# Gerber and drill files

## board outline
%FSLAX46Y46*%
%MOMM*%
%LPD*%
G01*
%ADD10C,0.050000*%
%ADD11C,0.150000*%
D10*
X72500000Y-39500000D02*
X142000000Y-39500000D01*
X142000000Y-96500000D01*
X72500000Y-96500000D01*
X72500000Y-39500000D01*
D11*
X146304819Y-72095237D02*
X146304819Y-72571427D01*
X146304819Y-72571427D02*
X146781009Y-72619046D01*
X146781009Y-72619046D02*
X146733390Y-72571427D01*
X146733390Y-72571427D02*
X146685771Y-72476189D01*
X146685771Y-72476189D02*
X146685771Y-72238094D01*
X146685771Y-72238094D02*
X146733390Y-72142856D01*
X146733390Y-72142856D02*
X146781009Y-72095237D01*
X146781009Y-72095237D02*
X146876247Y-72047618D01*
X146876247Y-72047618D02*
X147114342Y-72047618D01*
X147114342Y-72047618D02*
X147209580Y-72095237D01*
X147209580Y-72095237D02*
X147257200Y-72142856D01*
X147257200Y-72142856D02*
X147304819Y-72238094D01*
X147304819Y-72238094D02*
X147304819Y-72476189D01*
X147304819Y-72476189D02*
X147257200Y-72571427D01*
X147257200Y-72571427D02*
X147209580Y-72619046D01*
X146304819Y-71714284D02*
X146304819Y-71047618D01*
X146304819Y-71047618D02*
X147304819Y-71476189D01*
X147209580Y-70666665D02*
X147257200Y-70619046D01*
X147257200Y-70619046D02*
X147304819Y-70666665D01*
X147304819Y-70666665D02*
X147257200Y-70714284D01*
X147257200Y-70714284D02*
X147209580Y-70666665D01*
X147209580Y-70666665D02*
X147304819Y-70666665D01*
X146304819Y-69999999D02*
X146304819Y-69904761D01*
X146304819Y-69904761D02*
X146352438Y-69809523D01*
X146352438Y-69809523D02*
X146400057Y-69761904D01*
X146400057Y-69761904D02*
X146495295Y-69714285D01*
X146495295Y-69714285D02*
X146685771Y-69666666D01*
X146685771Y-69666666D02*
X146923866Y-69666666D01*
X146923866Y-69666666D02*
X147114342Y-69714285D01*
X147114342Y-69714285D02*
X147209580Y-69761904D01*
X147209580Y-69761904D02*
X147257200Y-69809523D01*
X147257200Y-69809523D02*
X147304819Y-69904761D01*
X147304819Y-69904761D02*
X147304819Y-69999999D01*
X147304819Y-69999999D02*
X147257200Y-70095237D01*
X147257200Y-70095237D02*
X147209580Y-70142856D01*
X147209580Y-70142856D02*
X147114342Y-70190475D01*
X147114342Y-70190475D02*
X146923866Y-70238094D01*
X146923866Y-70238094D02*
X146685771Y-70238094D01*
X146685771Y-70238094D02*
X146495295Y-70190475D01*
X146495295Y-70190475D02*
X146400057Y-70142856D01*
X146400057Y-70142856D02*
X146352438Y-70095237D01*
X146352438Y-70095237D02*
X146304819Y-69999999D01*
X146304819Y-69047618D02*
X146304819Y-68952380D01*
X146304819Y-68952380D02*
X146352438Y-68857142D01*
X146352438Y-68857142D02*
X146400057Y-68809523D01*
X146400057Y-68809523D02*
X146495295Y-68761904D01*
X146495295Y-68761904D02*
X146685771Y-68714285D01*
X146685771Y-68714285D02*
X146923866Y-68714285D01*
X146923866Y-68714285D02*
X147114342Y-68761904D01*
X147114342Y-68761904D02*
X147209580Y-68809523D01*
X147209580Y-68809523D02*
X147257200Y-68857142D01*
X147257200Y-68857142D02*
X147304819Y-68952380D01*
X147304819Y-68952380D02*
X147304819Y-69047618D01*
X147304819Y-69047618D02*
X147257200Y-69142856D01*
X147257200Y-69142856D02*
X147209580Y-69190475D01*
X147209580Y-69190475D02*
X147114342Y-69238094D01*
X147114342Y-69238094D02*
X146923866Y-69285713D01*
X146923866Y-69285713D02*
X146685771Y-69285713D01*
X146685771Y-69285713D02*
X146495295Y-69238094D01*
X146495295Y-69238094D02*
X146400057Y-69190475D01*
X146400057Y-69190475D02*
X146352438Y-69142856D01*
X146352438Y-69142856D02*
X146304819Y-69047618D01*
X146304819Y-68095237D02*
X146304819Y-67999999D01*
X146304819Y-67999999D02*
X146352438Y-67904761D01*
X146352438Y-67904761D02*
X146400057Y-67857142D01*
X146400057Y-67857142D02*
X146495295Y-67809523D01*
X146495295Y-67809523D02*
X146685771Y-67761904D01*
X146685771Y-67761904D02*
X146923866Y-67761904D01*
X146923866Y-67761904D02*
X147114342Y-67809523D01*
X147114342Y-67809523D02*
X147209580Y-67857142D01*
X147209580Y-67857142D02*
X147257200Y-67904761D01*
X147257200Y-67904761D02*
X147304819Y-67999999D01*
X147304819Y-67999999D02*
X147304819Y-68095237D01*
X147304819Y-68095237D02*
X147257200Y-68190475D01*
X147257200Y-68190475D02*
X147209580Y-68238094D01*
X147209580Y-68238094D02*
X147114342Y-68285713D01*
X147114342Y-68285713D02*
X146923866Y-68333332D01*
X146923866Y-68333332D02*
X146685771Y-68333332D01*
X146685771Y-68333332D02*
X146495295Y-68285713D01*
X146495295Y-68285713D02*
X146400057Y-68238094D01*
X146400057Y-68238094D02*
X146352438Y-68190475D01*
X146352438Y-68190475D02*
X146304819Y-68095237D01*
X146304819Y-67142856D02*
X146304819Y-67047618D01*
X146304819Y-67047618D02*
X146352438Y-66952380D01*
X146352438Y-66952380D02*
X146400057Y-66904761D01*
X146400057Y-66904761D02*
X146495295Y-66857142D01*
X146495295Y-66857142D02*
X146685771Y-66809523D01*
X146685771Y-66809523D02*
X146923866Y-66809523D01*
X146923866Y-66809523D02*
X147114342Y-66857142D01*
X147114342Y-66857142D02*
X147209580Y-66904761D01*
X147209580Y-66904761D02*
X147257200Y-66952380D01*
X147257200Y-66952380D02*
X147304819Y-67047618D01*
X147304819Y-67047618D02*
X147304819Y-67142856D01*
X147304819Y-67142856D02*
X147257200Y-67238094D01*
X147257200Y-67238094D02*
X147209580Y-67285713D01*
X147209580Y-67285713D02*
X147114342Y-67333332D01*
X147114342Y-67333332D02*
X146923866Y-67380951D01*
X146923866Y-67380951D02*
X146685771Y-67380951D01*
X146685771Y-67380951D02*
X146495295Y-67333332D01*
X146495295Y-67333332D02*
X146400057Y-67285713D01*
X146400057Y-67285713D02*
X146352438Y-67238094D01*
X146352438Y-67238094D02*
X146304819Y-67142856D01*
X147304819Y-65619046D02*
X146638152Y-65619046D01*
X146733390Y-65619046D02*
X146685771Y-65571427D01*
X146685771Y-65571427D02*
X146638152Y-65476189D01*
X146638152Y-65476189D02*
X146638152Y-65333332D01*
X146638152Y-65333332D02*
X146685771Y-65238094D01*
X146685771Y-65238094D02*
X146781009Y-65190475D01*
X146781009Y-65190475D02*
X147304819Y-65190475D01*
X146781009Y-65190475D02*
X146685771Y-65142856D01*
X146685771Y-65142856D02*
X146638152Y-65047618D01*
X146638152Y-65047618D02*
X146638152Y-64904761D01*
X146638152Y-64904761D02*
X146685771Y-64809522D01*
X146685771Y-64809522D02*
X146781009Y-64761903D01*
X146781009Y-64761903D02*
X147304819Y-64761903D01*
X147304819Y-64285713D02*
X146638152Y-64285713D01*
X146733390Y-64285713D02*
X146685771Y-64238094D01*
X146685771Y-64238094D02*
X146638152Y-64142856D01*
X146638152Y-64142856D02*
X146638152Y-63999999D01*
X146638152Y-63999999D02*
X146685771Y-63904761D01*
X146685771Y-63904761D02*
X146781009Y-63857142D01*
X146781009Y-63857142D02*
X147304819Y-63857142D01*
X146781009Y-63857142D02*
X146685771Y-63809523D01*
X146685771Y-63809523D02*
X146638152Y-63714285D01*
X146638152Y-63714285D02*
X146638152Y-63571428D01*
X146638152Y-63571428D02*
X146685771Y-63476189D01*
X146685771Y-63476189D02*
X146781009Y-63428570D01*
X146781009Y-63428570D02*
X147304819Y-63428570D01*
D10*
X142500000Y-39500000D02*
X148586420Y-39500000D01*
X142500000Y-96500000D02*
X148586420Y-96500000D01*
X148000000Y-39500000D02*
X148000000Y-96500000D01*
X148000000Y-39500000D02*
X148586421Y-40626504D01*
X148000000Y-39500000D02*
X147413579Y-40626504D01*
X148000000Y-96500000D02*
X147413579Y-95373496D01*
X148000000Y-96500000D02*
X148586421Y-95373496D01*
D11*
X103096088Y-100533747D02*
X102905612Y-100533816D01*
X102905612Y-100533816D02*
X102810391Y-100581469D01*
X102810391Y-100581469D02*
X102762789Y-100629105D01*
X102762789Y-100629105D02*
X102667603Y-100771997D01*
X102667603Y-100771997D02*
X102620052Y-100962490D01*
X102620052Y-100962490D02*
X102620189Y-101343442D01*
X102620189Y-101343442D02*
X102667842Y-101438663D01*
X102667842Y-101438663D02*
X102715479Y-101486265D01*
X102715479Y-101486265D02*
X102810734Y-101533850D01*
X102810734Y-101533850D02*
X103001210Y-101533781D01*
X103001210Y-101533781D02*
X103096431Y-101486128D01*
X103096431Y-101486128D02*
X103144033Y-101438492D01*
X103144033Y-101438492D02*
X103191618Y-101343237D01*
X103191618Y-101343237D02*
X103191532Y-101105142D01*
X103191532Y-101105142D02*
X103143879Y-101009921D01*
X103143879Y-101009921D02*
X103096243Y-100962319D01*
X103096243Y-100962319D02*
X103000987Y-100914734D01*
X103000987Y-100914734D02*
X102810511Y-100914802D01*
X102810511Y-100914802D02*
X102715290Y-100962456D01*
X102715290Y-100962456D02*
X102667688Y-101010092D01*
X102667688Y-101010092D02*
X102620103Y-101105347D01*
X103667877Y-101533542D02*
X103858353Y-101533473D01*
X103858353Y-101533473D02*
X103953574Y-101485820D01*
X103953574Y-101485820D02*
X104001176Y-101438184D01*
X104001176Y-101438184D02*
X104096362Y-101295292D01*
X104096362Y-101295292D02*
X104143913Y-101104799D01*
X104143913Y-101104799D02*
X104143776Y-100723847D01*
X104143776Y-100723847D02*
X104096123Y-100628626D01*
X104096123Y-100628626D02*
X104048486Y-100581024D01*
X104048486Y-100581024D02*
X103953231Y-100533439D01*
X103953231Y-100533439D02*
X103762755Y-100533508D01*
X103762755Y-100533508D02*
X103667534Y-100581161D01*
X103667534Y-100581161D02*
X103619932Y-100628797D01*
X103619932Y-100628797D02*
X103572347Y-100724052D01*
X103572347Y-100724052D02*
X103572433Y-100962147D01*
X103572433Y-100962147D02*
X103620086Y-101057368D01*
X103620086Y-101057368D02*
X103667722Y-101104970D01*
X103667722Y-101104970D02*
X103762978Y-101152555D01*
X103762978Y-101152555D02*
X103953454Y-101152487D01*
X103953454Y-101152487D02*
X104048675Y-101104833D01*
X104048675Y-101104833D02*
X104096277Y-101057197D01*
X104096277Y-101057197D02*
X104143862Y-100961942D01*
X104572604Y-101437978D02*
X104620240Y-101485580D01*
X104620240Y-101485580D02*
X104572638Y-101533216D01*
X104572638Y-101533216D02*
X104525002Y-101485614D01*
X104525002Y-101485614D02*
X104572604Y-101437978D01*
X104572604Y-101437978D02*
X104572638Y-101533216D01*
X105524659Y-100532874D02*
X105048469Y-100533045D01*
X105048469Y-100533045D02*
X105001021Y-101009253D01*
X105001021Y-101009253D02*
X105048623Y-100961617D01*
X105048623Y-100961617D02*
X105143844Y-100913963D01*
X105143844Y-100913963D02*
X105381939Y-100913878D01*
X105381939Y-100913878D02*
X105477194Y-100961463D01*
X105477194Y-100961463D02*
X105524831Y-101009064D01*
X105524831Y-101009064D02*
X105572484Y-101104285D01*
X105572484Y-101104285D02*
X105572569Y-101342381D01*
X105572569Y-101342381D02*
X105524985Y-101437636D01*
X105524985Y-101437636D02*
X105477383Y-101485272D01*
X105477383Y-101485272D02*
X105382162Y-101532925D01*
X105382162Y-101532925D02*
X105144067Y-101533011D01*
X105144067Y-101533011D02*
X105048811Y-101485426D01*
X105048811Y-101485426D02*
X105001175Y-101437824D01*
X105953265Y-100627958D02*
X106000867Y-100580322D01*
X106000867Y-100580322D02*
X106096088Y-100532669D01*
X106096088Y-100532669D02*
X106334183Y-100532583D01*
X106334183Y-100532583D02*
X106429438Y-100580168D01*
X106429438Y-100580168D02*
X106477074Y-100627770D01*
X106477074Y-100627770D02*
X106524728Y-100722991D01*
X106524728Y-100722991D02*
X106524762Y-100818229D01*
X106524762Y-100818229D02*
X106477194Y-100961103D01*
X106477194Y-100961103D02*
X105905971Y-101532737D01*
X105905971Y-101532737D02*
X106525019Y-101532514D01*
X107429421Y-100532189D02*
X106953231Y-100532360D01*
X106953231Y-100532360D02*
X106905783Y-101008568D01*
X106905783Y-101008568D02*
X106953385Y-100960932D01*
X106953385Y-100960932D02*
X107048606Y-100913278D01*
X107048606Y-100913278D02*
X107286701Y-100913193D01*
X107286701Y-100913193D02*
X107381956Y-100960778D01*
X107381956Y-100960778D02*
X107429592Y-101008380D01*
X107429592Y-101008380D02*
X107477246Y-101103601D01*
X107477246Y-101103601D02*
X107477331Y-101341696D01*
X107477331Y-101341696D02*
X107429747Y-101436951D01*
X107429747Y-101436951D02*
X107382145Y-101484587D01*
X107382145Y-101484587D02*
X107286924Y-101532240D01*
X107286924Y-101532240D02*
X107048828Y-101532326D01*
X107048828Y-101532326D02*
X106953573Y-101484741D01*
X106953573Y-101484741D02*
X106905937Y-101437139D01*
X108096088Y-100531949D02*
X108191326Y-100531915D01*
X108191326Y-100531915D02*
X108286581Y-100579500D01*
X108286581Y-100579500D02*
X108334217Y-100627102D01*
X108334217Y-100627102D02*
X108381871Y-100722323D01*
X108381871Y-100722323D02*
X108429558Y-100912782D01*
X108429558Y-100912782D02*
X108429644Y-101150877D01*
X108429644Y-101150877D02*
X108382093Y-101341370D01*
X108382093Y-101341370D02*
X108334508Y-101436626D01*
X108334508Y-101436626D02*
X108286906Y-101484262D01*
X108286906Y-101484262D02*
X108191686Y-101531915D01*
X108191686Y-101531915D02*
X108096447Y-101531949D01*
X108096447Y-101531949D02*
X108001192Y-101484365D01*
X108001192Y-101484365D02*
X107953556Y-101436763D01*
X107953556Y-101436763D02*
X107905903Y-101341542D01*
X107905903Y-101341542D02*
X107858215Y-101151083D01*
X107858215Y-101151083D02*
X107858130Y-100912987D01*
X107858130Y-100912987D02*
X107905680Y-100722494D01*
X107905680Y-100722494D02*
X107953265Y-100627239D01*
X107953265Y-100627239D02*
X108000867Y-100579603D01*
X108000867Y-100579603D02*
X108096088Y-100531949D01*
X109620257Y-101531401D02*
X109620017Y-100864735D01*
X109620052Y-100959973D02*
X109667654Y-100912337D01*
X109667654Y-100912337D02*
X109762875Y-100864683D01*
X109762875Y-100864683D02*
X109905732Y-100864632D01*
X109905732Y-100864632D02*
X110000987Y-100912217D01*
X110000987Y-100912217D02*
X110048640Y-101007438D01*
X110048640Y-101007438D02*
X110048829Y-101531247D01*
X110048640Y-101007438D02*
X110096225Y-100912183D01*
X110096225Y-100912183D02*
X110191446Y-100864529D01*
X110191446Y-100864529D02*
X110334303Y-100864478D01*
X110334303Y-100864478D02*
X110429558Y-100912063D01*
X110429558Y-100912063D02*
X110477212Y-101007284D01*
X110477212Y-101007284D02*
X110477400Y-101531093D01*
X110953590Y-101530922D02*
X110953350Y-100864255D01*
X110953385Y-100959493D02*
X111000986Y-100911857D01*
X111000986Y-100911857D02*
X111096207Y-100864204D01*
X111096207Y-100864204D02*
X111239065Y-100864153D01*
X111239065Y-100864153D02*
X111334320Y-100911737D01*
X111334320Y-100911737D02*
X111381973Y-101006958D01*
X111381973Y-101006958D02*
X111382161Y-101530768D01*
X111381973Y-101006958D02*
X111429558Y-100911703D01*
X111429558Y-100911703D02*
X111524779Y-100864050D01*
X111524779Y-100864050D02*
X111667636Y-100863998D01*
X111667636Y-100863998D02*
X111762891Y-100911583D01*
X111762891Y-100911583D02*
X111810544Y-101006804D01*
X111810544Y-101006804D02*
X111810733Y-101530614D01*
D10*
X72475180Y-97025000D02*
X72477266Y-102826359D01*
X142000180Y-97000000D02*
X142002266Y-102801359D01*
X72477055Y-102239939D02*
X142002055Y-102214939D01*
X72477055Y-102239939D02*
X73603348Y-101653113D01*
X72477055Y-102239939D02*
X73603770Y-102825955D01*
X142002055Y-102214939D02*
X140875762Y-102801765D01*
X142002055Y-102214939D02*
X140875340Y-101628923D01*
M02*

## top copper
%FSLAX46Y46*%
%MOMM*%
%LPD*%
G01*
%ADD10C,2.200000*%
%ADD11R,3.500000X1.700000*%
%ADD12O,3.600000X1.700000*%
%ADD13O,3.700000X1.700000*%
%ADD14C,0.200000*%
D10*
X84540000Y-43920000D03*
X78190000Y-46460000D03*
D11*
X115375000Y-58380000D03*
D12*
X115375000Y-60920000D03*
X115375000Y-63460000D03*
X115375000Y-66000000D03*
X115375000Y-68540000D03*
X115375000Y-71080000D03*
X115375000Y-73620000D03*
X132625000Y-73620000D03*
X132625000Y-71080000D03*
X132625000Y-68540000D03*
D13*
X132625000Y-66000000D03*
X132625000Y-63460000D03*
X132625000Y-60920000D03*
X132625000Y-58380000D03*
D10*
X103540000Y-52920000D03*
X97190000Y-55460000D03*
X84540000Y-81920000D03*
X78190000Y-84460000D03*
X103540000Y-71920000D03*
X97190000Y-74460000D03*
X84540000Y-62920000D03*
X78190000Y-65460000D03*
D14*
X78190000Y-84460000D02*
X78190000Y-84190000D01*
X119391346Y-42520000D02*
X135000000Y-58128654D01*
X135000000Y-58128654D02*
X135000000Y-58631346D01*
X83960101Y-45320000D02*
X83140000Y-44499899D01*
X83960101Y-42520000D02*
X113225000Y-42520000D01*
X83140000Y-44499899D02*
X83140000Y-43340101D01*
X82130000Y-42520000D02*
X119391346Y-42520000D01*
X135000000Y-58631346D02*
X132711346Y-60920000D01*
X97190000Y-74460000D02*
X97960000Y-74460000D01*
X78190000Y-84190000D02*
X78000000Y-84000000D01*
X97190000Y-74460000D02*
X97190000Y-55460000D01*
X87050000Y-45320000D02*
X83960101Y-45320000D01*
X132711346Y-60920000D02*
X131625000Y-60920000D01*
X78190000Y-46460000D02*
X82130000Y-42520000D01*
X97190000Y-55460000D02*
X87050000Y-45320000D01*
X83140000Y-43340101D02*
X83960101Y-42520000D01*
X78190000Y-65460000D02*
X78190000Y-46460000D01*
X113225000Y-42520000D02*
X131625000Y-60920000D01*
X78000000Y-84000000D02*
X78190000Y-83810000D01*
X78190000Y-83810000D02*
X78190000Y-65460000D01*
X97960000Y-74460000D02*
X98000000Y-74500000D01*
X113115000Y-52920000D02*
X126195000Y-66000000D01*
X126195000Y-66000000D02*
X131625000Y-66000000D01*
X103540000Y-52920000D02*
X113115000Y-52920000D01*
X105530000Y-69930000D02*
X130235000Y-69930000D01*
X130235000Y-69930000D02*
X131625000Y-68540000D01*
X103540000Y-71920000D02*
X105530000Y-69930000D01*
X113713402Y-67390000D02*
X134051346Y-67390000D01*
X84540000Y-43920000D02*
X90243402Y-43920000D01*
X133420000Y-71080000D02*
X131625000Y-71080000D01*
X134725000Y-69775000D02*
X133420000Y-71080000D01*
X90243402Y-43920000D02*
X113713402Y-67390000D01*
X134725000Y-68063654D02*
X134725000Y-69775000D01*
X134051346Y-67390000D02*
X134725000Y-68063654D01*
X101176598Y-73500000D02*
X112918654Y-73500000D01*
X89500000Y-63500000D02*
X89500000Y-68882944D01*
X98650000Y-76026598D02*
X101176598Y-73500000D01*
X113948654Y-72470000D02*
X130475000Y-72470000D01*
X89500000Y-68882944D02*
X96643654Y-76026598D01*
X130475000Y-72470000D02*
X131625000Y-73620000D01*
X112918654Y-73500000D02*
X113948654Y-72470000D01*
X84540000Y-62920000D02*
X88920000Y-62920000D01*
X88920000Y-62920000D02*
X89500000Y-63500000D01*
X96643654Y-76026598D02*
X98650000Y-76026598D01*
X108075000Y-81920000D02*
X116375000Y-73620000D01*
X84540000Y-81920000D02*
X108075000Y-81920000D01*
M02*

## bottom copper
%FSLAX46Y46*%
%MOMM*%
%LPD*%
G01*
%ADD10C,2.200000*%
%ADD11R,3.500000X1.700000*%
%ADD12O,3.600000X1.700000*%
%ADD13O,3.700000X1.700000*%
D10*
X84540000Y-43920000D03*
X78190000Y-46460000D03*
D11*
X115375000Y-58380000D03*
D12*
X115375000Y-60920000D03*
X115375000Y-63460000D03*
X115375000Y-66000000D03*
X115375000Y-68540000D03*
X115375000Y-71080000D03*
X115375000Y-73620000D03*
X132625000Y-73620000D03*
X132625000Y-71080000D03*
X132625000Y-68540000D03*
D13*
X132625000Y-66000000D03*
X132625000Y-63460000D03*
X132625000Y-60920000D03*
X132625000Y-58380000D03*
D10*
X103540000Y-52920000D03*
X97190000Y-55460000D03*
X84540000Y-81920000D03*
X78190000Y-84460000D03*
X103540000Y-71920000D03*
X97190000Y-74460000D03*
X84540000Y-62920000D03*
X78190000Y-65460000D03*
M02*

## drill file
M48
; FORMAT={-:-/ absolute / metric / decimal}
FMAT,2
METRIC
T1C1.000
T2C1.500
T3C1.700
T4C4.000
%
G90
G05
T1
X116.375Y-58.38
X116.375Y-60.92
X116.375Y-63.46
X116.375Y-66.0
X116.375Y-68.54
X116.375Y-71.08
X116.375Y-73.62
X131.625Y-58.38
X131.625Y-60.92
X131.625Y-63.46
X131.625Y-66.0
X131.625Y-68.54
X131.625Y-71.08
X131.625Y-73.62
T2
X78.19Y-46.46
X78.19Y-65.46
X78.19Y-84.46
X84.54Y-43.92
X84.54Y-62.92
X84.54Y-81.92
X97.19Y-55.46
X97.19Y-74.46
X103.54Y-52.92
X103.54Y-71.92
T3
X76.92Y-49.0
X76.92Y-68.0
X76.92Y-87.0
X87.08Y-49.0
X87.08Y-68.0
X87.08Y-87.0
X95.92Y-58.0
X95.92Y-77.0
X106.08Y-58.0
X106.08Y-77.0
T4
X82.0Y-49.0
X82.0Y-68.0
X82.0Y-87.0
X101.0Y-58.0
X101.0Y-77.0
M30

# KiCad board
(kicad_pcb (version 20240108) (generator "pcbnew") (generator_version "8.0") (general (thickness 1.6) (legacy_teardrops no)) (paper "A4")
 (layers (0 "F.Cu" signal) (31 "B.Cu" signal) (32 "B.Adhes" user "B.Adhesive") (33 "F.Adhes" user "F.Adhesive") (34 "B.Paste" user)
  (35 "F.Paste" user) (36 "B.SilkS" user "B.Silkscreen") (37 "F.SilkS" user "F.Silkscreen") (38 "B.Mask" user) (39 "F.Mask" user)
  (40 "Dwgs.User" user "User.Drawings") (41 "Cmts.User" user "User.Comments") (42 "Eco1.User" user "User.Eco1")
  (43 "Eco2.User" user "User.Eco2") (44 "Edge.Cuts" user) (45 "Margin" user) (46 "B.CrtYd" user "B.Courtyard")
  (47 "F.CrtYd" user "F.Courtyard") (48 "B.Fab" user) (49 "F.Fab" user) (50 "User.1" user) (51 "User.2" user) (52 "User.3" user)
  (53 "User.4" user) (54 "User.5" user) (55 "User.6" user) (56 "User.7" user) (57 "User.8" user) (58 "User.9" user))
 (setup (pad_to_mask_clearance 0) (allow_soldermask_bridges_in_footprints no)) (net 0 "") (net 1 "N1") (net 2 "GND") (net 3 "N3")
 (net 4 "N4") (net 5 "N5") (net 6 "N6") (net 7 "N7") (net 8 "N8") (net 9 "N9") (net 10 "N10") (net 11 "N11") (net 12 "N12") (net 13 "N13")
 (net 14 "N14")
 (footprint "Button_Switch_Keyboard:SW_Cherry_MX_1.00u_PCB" (layer "F.Cu") (at 84.54 43.92)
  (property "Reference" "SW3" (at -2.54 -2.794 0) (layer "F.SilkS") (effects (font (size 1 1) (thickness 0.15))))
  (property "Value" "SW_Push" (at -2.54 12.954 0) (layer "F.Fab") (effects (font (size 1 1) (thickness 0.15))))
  (pad "" np_thru_hole circle (at -7.62 5.08) (size 1.7 1.7) (drill 1.7) (layers "*.Cu" "*.Mask"))
  (pad "" np_thru_hole circle (at -2.54 5.08) (size 4 4) (drill 4) (layers "*.Cu" "*.Mask"))
  (pad "" np_thru_hole circle (at 2.54 5.08) (size 1.7 1.7) (drill 1.7) (layers "*.Cu" "*.Mask"))
  (pad "1" thru_hole circle (at 0 0) (size 2.2 2.2) (drill 1.5) (layers "*.Cu" "*.Mask") (remove_unused_layers no) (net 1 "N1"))
  (pad "2" thru_hole circle (at -6.35 2.54) (size 2.2 2.2) (drill 1.5) (layers "*.Cu" "*.Mask") (remove_unused_layers no) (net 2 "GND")))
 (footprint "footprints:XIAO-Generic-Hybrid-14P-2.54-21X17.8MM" (layer "F.Cu") (at 124 66)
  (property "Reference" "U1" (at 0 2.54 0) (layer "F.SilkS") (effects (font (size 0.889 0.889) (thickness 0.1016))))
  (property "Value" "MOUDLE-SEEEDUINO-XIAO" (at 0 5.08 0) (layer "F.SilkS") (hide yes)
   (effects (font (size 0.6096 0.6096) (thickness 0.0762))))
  (pad "1" thru_hole rect (at -7.625 -7.62) (size 3.5 1.7) (drill 1 (offset -1 0)) (layers "*.Cu" "*.Mask") (remove_unused_layers no)
   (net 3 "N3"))
  (pad "2" thru_hole oval (at -7.625 -5.08) (size 3.6 1.7) (drill 1 (offset -1 0)) (layers "*.Cu" "*.Mask") (remove_unused_layers no)
   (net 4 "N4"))
  (pad "3" thru_hole oval (at -7.625 -2.54) (size 3.6 1.7) (drill 1 (offset -1 0)) (layers "*.Cu" "*.Mask") (remove_unused_layers no)
   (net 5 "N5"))
  (pad "4" thru_hole oval (at -7.625 0) (size 3.6 1.7) (drill 1 (offset -1 0)) (layers "*.Cu" "*.Mask") (remove_unused_layers no)
   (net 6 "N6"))
  (pad "5" thru_hole oval (at -7.625 2.54) (size 3.6 1.7) (drill 1 (offset -1 0)) (layers "*.Cu" "*.Mask") (remove_unused_layers no)
   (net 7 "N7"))
  (pad "6" thru_hole oval (at -7.625 5.08 180) (size 3.6 1.7) (drill 1 (offset 1 0)) (layers "*.Cu" "*.Mask") (remove_unused_layers no)
   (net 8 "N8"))
  (pad "7" thru_hole oval (at -7.625 7.62) (size 3.6 1.7) (drill 1 (offset -1 0)) (layers "*.Cu" "*.Mask") (remove_unused_layers no)
   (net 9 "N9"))
  (pad "8" thru_hole oval (at 7.625 7.62) (size 3.6 1.7) (drill 1 (offset 1 0)) (layers "*.Cu" "*.Mask") (remove_unused_layers no)
   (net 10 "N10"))
  (pad "9" thru_hole oval (at 7.625 5.08) (size 3.6 1.7) (drill 1 (offset 1 0)) (layers "*.Cu" "*.Mask") (remove_unused_layers no)
   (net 1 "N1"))
  (pad "10" thru_hole oval (at 7.625 2.54) (size 3.6 1.7) (drill 1 (offset 1 0)) (layers "*.Cu" "*.Mask") (remove_unused_layers no)
   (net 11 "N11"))
  (pad "11" thru_hole oval (at 7.625 0) (size 3.7 1.7) (drill 1 (offset 1 0)) (layers "*.Cu" "*.Mask") (remove_unused_layers no)
   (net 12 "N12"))
  (pad "12" thru_hole oval (at 7.625 -2.54) (size 3.7 1.7) (drill 1 (offset 1 0)) (layers "*.Cu" "*.Mask") (remove_unused_layers no)
   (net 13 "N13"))
  (pad "13" thru_hole oval (at 7.625 -5.08) (size 3.7 1.7) (drill 1 (offset 1 0)) (layers "*.Cu" "*.Mask") (remove_unused_layers no)
   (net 2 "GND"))
  (pad "14" thru_hole oval (at 7.625 -7.62) (size 3.7 1.7) (drill 1 (offset 1 0)) (layers "*.Cu" "*.Mask") (remove_unused_layers no)
   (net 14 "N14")))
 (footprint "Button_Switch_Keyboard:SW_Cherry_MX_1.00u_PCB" (layer "F.Cu") (at 103.54 52.92)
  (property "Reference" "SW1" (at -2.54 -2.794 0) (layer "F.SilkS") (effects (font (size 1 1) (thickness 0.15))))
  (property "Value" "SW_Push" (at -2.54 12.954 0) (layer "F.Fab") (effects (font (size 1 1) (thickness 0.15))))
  (pad "" np_thru_hole circle (at -7.62 5.08) (size 1.7 1.7) (drill 1.7) (layers "*.Cu" "*.Mask"))
  (pad "" np_thru_hole circle (at -2.54 5.08) (size 4 4) (drill 4) (layers "*.Cu" "*.Mask"))
  (pad "" np_thru_hole circle (at 2.54 5.08) (size 1.7 1.7) (drill 1.7) (layers "*.Cu" "*.Mask"))
  (pad "1" thru_hole circle (at 0 0) (size 2.2 2.2) (drill 1.5) (layers "*.Cu" "*.Mask") (remove_unused_layers no) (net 12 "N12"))
  (pad "2" thru_hole circle (at -6.35 2.54) (size 2.2 2.2) (drill 1.5) (layers "*.Cu" "*.Mask") (remove_unused_layers no) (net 2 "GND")))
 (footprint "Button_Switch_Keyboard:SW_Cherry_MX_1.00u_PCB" (layer "F.Cu") (at 84.54 81.92)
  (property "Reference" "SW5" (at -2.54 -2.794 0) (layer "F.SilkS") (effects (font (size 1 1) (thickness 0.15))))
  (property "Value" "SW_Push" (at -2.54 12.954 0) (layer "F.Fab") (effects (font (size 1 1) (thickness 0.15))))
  (pad "" np_thru_hole circle (at -7.62 5.08) (size 1.7 1.7) (drill 1.7) (layers "*.Cu" "*.Mask"))
  (pad "" np_thru_hole circle (at -2.54 5.08) (size 4 4) (drill 4) (layers "*.Cu" "*.Mask"))
  (pad "" np_thru_hole circle (at 2.54 5.08) (size 1.7 1.7) (drill 1.7) (layers "*.Cu" "*.Mask"))
  (pad "1" thru_hole circle (at 0 0) (size 2.2 2.2) (drill 1.5) (layers "*.Cu" "*.Mask") (remove_unused_layers no) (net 9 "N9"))
  (pad "2" thru_hole circle (at -6.35 2.54) (size 2.2 2.2) (drill 1.5) (layers "*.Cu" "*.Mask") (remove_unused_layers no) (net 2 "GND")))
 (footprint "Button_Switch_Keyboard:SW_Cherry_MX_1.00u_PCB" (layer "F.Cu") (at 103.54 71.92)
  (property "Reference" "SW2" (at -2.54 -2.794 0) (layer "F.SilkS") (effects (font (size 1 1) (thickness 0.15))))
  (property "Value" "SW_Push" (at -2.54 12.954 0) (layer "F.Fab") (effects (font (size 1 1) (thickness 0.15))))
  (pad "" np_thru_hole circle (at -7.62 5.08) (size 1.7 1.7) (drill 1.7) (layers "*.Cu" "*.Mask"))
  (pad "" np_thru_hole circle (at -2.54 5.08) (size 4 4) (drill 4) (layers "*.Cu" "*.Mask"))
  (pad "" np_thru_hole circle (at 2.54 5.08) (size 1.7 1.7) (drill 1.7) (layers "*.Cu" "*.Mask"))
  (pad "1" thru_hole circle (at 0 0) (size 2.2 2.2) (drill 1.5) (layers "*.Cu" "*.Mask") (remove_unused_layers no) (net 11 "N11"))
  (pad "2" thru_hole circle (at -6.35 2.54) (size 2.2 2.2) (drill 1.5) (layers "*.Cu" "*.Mask") (remove_unused_layers no) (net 2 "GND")))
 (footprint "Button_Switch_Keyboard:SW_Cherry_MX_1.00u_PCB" (layer "F.Cu") (at 84.54 62.92)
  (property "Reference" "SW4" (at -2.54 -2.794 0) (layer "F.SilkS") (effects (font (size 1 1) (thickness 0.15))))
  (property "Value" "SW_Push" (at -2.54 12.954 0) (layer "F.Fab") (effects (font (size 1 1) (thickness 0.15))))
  (pad "" np_thru_hole circle (at -7.62 5.08) (size 1.7 1.7) (drill 1.7) (layers "*.Cu" "*.Mask"))
  (pad "" np_thru_hole circle (at -2.54 5.08) (size 4 4) (drill 4) (layers "*.Cu" "*.Mask"))
  (pad "" np_thru_hole circle (at 2.54 5.08) (size 1.7 1.7) (drill 1.7) (layers "*.Cu" "*.Mask"))
  (pad "1" thru_hole circle (at 0 0) (size 2.2 2.2) (drill 1.5) (layers "*.Cu" "*.Mask") (remove_unused_layers no) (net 10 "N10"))
  (pad "2" thru_hole circle (at -6.35 2.54) (size 2.2 2.2) (drill 1.5) (layers "*.Cu" "*.Mask") (remove_unused_layers no) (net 2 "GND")))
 (gr_rect (start 72.5 39.5) (end 142 96.5) (stroke (width 0.05) (type default)) (fill none) (layer "Edge.Cuts"))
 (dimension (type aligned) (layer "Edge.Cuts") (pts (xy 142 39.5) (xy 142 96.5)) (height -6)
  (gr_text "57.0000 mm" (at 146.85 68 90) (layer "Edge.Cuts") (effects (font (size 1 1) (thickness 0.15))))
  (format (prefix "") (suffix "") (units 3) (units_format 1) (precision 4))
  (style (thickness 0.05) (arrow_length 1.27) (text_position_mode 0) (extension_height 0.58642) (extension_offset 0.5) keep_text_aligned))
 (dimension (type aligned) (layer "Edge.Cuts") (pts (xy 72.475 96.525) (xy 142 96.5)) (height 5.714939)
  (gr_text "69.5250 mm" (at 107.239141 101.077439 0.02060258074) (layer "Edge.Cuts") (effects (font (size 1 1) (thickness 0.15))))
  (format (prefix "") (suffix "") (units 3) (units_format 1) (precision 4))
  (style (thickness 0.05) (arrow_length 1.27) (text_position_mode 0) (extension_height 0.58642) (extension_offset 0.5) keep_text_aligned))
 (segment (start 78.19 84.46) (end 78.19 84.19) (width 0.2) (layer "F.Cu") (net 2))
 (segment (start 119.391346 42.52) (end 135 58.128654) (width 0.2) (layer "F.Cu") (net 2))
 (segment (start 135 58.128654) (end 135 58.631346) (width 0.2) (layer "F.Cu") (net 2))
 (segment (start 83.960101 45.32) (end 83.14 44.499899) (width 0.2) (layer "F.Cu") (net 2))
 (segment (start 83.960101 42.52) (end 113.225 42.52) (width 0.2) (layer "F.Cu") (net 2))
 (segment (start 83.14 44.499899) (end 83.14 43.340101) (width 0.2) (layer "F.Cu") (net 2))
 (segment (start 82.13 42.52) (end 119.391346 42.52) (width 0.2) (layer "F.Cu") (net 2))
 (segment (start 135 58.631346) (end 132.711346 60.92) (width 0.2) (layer "F.Cu") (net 2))
 (segment (start 97.19 74.46) (end 97.96 74.46) (width 0.2) (layer "F.Cu") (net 2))
 (segment (start 78.19 84.19) (end 78 84) (width 0.2) (layer "F.Cu") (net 2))
 (segment (start 97.19 74.46) (end 97.19 55.46) (width 0.2) (layer "F.Cu") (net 2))
 (segment (start 87.05 45.32) (end 83.960101 45.32) (width 0.2) (layer "F.Cu") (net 2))
 (segment (start 132.711346 60.92) (end 131.625 60.92) (width 0.2) (layer "F.Cu") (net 2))
 (segment (start 78.19 46.46) (end 82.13 42.52) (width 0.2) (layer "F.Cu") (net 2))
 (segment (start 97.19 55.46) (end 87.05 45.32) (width 0.2) (layer "F.Cu") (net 2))
 (segment (start 83.14 43.340101) (end 83.960101 42.52) (width 0.2) (layer "F.Cu") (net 2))
 (segment (start 78.19 65.46) (end 78.19 46.46) (width 0.2) (layer "F.Cu") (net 2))
 (segment (start 113.225 42.52) (end 131.625 60.92) (width 0.2) (layer "F.Cu") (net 2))
 (segment (start 78 84) (end 78.19 83.81) (width 0.2) (layer "F.Cu") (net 2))
 (segment (start 78.19 83.81) (end 78.19 65.46) (width 0.2) (layer "F.Cu") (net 2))
 (segment (start 97.96 74.46) (end 98 74.5) (width 0.2) (layer "F.Cu") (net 2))
 (segment (start 113.115 52.92) (end 126.195 66) (width 0.2) (layer "F.Cu") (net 12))
 (segment (start 126.195 66) (end 131.625 66) (width 0.2) (layer "F.Cu") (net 12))
 (segment (start 103.54 52.92) (end 113.115 52.92) (width 0.2) (layer "F.Cu") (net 12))
 (segment (start 105.53 69.93) (end 130.235 69.93) (width 0.2) (layer "F.Cu") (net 11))
 (segment (start 130.235 69.93) (end 131.625 68.54) (width 0.2) (layer "F.Cu") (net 11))
 (segment (start 103.54 71.92) (end 105.53 69.93) (width 0.2) (layer "F.Cu") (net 11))
 (segment (start 113.713402 67.39) (end 134.051346 67.39) (width 0.2) (layer "F.Cu") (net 1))
 (segment (start 84.54 43.92) (end 90.243402 43.92) (width 0.2) (layer "F.Cu") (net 1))
 (segment (start 133.42 71.08) (end 131.625 71.08) (width 0.2) (layer "F.Cu") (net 1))
 (segment (start 134.725 69.775) (end 133.42 71.08) (width 0.2) (layer "F.Cu") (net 1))
 (segment (start 90.243402 43.92) (end 113.713402 67.39) (width 0.2) (layer "F.Cu") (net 1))
 (segment (start 134.725 68.063654) (end 134.725 69.775) (width 0.2) (layer "F.Cu") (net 1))
 (segment (start 134.051346 67.39) (end 134.725 68.063654) (width 0.2) (layer "F.Cu") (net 1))
 (segment (start 101.176598 73.5) (end 112.918654 73.5) (width 0.2) (layer "F.Cu") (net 10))
 (segment (start 89.5 63.5) (end 89.5 68.882944) (width 0.2) (layer "F.Cu") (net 10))
 (segment (start 98.65 76.026598) (end 101.176598 73.5) (width 0.2) (layer "F.Cu") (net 10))
 (segment (start 113.948654 72.47) (end 130.475 72.47) (width 0.2) (layer "F.Cu") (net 10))
 (segment (start 89.5 68.882944) (end 96.643654 76.026598) (width 0.2) (layer "F.Cu") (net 10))
 (segment (start 130.475 72.47) (end 131.625 73.62) (width 0.2) (layer "F.Cu") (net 10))
 (segment (start 112.918654 73.5) (end 113.948654 72.47) (width 0.2) (layer "F.Cu") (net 10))
 (segment (start 84.54 62.92) (end 88.92 62.92) (width 0.2) (layer "F.Cu") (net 10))
 (segment (start 88.92 62.92) (end 89.5 63.5) (width 0.2) (layer "F.Cu") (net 10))
 (segment (start 96.643654 76.026598) (end 98.65 76.026598) (width 0.2) (layer "F.Cu") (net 10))
 (segment (start 108.075 81.92) (end 116.375 73.62) (width 0.2) (layer "F.Cu") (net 9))
 (segment (start 84.54 81.92) (end 108.075 81.92) (width 0.2) (layer "F.Cu") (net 9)))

